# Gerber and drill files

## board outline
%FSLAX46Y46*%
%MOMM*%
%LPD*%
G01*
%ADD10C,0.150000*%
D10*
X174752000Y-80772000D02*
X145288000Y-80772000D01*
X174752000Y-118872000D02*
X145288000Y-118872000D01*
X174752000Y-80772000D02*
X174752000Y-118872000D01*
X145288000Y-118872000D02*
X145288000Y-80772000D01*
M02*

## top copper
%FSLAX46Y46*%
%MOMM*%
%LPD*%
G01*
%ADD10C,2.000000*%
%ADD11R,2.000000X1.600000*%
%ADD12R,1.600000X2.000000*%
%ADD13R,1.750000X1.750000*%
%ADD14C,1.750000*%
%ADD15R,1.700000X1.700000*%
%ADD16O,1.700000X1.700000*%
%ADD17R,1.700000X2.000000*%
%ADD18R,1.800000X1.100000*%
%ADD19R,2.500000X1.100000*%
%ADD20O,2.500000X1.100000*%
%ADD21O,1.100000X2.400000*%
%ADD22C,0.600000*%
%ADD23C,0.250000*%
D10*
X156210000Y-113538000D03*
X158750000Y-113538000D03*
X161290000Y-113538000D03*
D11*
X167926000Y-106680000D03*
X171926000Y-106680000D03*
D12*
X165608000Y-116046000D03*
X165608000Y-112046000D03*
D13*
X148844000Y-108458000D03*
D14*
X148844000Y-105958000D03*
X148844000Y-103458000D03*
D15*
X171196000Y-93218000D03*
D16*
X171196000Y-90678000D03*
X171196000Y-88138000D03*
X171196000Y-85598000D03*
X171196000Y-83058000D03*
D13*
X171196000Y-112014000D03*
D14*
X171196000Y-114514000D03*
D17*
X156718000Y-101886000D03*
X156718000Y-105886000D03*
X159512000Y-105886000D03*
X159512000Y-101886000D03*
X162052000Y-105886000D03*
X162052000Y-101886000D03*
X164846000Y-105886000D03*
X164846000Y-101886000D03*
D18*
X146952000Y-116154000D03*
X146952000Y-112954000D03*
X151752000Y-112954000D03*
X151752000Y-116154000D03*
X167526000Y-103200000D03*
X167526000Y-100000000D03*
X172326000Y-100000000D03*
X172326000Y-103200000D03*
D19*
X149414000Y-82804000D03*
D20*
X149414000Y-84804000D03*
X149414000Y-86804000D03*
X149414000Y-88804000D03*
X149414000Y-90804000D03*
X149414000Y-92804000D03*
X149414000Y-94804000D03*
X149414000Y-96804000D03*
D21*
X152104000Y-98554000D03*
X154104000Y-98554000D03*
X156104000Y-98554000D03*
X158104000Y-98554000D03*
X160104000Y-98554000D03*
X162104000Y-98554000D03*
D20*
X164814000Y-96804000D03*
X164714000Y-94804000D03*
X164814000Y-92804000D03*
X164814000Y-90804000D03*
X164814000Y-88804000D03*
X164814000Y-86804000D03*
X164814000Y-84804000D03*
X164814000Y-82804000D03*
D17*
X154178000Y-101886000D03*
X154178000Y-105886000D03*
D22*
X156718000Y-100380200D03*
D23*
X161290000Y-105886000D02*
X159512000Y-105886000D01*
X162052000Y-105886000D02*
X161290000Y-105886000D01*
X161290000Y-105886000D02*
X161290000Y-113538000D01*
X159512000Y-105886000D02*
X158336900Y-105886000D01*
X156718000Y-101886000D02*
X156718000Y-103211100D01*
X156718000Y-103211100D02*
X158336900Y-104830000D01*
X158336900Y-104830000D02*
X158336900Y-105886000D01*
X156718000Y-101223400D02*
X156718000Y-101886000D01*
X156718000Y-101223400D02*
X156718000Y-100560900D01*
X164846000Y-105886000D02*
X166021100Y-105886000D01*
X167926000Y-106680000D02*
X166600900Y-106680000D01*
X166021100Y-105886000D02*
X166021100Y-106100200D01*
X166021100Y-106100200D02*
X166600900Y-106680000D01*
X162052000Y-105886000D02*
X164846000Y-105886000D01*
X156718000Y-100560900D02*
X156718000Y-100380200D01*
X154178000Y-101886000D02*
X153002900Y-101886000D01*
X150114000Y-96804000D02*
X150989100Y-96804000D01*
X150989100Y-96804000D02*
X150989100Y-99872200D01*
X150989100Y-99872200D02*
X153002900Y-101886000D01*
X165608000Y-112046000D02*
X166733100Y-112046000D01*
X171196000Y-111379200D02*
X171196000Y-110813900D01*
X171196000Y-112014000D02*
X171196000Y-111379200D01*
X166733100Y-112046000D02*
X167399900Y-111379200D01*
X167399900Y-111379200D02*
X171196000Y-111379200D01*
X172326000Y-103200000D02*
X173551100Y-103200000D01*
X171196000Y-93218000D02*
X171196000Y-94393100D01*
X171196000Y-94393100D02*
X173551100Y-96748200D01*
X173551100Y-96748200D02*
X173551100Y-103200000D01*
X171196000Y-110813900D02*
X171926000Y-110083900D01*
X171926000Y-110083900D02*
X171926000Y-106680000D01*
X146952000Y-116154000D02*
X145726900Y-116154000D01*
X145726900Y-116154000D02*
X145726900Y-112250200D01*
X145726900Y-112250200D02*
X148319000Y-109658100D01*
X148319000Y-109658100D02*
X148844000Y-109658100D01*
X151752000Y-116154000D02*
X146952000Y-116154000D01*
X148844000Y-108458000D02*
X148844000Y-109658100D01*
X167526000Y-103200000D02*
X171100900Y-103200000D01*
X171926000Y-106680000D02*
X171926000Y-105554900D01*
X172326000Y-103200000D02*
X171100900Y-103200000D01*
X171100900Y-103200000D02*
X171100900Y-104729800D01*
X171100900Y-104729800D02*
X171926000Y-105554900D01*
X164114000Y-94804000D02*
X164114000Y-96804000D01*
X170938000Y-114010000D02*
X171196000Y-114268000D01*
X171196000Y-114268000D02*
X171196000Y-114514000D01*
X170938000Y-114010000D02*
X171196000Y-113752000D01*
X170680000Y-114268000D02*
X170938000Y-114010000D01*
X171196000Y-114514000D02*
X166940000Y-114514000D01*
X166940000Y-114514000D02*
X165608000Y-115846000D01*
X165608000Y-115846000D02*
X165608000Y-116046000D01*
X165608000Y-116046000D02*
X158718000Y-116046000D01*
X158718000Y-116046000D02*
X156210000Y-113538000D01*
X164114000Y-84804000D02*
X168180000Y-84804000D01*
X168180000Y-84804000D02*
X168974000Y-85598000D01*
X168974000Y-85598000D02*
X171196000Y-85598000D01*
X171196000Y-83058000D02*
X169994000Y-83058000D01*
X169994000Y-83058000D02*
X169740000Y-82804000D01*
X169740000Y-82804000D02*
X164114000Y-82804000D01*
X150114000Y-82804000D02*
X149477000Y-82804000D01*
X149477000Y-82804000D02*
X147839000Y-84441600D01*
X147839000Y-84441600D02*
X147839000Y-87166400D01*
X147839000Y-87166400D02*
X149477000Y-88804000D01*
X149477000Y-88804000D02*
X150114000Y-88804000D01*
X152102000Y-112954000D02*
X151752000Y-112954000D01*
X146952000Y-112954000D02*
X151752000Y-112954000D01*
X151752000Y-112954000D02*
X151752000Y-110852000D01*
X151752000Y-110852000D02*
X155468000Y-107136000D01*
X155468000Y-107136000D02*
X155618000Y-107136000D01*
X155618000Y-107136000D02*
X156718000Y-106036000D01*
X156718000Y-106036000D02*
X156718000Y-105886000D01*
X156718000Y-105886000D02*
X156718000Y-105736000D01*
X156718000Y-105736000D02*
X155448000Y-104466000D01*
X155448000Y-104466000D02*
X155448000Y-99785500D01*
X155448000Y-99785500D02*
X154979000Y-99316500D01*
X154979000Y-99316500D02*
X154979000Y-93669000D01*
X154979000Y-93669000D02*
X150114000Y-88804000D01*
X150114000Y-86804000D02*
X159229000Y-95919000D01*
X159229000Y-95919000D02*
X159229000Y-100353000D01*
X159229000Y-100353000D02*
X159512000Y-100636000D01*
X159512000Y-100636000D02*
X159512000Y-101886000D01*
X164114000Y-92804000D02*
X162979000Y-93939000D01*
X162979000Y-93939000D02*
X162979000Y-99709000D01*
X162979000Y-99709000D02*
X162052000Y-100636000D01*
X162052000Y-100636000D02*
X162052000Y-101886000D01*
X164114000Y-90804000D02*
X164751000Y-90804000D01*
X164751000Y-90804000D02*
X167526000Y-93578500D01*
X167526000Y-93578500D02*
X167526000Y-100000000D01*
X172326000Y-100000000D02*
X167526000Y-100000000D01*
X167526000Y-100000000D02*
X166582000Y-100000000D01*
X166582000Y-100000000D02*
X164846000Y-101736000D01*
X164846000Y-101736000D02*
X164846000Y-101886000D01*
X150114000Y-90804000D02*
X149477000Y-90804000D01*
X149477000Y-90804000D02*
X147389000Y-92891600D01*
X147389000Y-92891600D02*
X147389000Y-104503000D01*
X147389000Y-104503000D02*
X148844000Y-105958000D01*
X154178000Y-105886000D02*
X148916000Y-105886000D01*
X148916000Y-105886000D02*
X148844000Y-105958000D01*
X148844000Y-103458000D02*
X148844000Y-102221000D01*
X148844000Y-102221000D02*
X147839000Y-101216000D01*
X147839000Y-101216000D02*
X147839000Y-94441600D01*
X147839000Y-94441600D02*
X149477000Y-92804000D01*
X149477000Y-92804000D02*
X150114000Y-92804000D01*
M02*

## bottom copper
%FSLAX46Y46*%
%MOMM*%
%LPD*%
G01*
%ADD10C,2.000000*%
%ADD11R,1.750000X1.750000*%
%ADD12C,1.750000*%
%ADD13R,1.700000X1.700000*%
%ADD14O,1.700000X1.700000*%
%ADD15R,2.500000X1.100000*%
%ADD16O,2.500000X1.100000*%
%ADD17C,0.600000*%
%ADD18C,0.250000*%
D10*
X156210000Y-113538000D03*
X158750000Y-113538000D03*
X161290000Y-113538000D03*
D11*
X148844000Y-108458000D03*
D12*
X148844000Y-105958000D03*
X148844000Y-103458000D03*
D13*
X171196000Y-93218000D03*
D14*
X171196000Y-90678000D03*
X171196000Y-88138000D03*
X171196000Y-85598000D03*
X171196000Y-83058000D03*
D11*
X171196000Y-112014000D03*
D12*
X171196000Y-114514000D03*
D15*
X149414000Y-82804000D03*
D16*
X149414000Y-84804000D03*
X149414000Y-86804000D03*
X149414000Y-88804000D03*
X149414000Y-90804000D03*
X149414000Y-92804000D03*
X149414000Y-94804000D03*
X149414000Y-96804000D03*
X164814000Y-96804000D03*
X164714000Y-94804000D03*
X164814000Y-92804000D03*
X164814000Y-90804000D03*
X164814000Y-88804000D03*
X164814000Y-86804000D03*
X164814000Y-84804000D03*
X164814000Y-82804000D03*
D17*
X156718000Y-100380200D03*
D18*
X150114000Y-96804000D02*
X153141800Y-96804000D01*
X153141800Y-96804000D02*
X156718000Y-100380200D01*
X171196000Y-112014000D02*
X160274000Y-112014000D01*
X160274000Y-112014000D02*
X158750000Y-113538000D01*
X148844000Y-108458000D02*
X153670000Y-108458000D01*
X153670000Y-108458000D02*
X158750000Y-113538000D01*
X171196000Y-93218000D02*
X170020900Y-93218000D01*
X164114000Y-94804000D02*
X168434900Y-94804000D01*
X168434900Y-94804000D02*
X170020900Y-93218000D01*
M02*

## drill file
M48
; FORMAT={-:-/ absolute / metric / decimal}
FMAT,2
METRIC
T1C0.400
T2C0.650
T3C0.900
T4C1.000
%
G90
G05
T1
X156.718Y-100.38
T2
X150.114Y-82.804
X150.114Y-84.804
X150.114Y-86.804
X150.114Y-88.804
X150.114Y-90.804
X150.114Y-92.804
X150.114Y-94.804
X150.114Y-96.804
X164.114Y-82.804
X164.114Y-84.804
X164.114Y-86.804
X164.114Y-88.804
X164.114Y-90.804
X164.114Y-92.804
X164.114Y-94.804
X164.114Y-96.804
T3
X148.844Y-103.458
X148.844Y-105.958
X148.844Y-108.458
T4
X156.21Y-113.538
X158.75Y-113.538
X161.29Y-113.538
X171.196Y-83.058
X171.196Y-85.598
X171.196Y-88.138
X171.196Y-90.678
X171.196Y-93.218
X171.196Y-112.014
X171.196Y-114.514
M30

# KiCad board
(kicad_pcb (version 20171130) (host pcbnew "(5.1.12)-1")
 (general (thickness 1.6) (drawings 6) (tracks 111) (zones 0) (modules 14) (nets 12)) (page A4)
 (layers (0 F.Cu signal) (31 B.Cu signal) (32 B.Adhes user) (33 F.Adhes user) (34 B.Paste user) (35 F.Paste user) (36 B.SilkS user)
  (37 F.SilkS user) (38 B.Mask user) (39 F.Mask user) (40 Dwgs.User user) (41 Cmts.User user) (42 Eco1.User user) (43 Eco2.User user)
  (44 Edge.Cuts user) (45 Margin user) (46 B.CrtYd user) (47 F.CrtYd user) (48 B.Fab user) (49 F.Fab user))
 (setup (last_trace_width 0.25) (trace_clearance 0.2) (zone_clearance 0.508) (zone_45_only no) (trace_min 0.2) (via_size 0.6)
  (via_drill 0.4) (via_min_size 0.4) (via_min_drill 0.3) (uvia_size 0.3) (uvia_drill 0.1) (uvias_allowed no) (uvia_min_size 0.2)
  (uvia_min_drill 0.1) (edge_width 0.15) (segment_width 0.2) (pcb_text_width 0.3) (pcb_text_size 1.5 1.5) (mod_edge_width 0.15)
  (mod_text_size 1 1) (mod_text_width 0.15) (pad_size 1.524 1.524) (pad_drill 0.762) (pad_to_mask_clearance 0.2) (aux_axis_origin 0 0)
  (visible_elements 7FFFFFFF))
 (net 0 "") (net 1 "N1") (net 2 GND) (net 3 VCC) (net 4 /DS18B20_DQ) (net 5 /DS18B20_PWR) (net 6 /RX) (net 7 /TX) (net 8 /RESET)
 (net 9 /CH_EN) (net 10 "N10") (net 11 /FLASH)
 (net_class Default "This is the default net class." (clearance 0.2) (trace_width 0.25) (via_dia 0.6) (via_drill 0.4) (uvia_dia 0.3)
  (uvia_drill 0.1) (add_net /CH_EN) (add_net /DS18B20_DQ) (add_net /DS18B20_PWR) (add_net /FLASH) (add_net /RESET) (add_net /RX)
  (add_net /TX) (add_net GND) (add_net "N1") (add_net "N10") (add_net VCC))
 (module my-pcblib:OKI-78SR (layer F.Cu) (at 158.75 113.538)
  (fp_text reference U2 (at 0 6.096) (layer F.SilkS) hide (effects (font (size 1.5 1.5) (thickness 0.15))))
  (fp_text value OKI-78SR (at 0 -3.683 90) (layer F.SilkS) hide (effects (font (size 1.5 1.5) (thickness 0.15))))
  (pad 1 thru_hole circle (at -2.54 0) (size 2 2) (drill 1) (layers *.Cu *.Mask F.SilkS) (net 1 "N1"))
  (pad 2 thru_hole circle (at 0 0) (size 2 2) (drill 1) (layers *.Cu *.Mask F.SilkS) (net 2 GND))
  (pad 3 thru_hole circle (at 2.54 0) (size 2 2) (drill 1) (layers *.Cu *.Mask F.SilkS) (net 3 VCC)))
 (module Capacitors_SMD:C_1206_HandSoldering (layer F.Cu) (at 169.926 106.68)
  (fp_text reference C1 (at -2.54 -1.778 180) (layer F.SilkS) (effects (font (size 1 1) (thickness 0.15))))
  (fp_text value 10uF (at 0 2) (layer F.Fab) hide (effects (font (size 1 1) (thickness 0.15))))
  (pad 1 smd rect (at -2 0) (size 2 1.6) (layers F.Cu F.Paste F.Mask) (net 3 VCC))
  (pad 2 smd rect (at 2 0) (size 2 1.6) (layers F.Cu F.Paste F.Mask) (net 2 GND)))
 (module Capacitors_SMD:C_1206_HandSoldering (layer F.Cu) (at 165.608 114.046 90)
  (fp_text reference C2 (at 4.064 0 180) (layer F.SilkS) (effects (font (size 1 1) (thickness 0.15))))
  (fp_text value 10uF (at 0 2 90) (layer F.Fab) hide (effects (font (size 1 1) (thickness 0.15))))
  (pad 1 smd rect (at -2 0 90) (size 2 1.6) (layers F.Cu F.Paste F.Mask) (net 1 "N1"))
  (pad 2 smd rect (at 2 0 90) (size 2 1.6) (layers F.Cu F.Paste F.Mask) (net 2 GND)))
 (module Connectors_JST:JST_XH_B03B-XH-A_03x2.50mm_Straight (layer F.Cu) (at 148.844 108.458 90)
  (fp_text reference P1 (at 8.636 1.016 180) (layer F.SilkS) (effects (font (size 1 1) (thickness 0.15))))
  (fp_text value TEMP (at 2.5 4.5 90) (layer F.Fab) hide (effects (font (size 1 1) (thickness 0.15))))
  (pad 1 thru_hole rect (at 0 0 90) (size 1.75 1.75) (drill 0.9) (layers *.Cu *.Mask) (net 2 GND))
  (pad 2 thru_hole circle (at 2.5 0 90) (size 1.75 1.75) (drill 0.9) (layers *.Cu *.Mask) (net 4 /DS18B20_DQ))
  (pad 3 thru_hole circle (at 5 0 90) (size 1.75 1.75) (drill 0.9) (layers *.Cu *.Mask) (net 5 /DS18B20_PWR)))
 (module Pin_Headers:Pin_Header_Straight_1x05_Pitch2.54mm (layer F.Cu) (at 171.196 93.218 180)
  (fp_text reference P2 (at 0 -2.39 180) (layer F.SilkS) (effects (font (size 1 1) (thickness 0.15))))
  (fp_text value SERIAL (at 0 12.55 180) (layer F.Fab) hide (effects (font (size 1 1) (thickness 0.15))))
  (pad 1 thru_hole rect (at 0 0 180) (size 1.7 1.7) (drill 1) (layers *.Cu *.Mask) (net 2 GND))
  (pad 2 thru_hole oval (at 0 2.54 180) (size 1.7 1.7) (drill 1) (layers *.Cu *.Mask))
  (pad 3 thru_hole oval (at 0 5.08 180) (size 1.7 1.7) (drill 1) (layers *.Cu *.Mask))
  (pad 4 thru_hole oval (at 0 7.62 180) (size 1.7 1.7) (drill 1) (layers *.Cu *.Mask) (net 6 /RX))
  (pad 5 thru_hole oval (at 0 10.16 180) (size 1.7 1.7) (drill 1) (layers *.Cu *.Mask) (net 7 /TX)))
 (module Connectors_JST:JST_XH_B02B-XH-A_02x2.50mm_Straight (layer F.Cu) (at 171.196 112.014 270)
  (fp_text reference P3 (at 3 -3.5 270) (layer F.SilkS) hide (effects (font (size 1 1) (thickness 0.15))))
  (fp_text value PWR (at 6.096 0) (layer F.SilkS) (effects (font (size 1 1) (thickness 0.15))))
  (pad 1 thru_hole rect (at 0 0 270) (size 1.75 1.75) (drill 1) (layers *.Cu *.Mask) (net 2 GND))
  (pad 2 thru_hole circle (at 2.5 0 270) (size 1.75 1.75) (drill 1) (layers *.Cu *.Mask) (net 1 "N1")))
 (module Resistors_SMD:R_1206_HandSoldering (layer F.Cu) (at 156.718 103.886 270)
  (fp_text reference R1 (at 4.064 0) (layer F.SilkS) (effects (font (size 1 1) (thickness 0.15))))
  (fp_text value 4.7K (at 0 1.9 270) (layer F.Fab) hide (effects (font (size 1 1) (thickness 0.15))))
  (pad 1 smd rect (at -2 0 270) (size 2 1.7) (layers F.Cu F.Paste F.Mask) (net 3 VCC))
  (pad 2 smd rect (at 2 0 270) (size 2 1.7) (layers F.Cu F.Paste F.Mask) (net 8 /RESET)))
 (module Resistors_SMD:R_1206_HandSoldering (layer F.Cu) (at 159.512 103.886 90)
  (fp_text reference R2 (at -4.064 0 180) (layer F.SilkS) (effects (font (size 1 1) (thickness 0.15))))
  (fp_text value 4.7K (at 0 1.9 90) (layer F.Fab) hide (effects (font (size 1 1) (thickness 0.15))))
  (pad 1 smd rect (at -2 0 90) (size 2 1.7) (layers F.Cu F.Paste F.Mask) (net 3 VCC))
  (pad 2 smd rect (at 2 0 90) (size 2 1.7) (layers F.Cu F.Paste F.Mask) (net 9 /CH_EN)))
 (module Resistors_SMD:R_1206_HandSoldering (layer F.Cu) (at 162.052 103.886 90)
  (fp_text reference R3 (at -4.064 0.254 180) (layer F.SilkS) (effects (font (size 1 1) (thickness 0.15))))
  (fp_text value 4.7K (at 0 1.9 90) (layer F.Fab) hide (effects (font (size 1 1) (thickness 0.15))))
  (pad 1 smd rect (at -2 0 90) (size 2 1.7) (layers F.Cu F.Paste F.Mask) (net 3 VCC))
  (pad 2 smd rect (at 2 0 90) (size 2 1.7) (layers F.Cu F.Paste F.Mask) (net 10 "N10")))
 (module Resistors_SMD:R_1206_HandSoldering (layer F.Cu) (at 164.846 103.886 90)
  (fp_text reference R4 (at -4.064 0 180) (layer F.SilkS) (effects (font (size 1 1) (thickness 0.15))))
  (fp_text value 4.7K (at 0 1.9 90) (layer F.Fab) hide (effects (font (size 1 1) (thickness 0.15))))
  (pad 1 smd rect (at -2 0 90) (size 2 1.7) (layers F.Cu F.Paste F.Mask) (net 3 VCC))
  (pad 2 smd rect (at 2 0 90) (size 2 1.7) (layers F.Cu F.Paste F.Mask) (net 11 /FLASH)))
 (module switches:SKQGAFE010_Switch (layer F.Cu) (at 149.352 114.554)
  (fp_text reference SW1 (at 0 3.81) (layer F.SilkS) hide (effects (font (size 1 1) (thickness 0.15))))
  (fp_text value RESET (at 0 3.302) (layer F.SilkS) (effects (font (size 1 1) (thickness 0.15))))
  (pad 3 smd rect (at -2.4 1.6) (size 1.8 1.1) (layers F.Cu F.Paste F.Mask) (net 2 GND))
  (pad 1 smd rect (at -2.4 -1.6) (size 1.8 1.1) (layers F.Cu F.Paste F.Mask) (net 8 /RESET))
  (pad 2 smd rect (at 2.4 -1.6) (size 1.8 1.1) (layers F.Cu F.Paste F.Mask) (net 8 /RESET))
  (pad 4 smd rect (at 2.4 1.6) (size 1.8 1.1) (layers F.Cu F.Paste F.Mask) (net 2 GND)))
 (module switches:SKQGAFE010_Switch (layer F.Cu) (at 169.926 101.6)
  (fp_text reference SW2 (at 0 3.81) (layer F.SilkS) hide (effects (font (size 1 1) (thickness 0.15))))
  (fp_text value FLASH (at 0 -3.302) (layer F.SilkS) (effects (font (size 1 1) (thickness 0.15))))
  (pad 3 smd rect (at -2.4 1.6) (size 1.8 1.1) (layers F.Cu F.Paste F.Mask) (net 2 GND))
  (pad 1 smd rect (at -2.4 -1.6) (size 1.8 1.1) (layers F.Cu F.Paste F.Mask) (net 11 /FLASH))
  (pad 2 smd rect (at 2.4 -1.6) (size 1.8 1.1) (layers F.Cu F.Paste F.Mask) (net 11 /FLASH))
  (pad 4 smd rect (at 2.4 1.6) (size 1.8 1.1) (layers F.Cu F.Paste F.Mask) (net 2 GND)))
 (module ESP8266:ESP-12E (layer F.Cu) (at 150.114 82.804)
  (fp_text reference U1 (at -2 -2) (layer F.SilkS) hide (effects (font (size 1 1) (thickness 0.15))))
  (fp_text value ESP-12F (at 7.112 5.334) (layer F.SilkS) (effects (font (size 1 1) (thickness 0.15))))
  (pad 1 thru_hole rect (at 0 0) (size 2.5 1.1) (drill 0.65 (offset -0.7 0)) (layers *.Cu *.Mask F.SilkS) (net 8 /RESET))
  (pad 2 thru_hole oval (at 0 2) (size 2.5 1.1) (drill 0.65 (offset -0.7 0)) (layers *.Cu *.Mask F.SilkS))
  (pad 3 thru_hole oval (at 0 4) (size 2.5 1.1) (drill 0.65 (offset -0.7 0)) (layers *.Cu *.Mask F.SilkS) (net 9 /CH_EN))
  (pad 4 thru_hole oval (at 0 6) (size 2.5 1.1) (drill 0.65 (offset -0.7 0)) (layers *.Cu *.Mask F.SilkS) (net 8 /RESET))
  (pad 5 thru_hole oval (at 0 8) (size 2.5 1.1) (drill 0.65 (offset -0.7 0)) (layers *.Cu *.Mask F.SilkS) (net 4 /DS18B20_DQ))
  (pad 6 thru_hole oval (at 0 10) (size 2.5 1.1) (drill 0.65 (offset -0.7 0)) (layers *.Cu *.Mask F.SilkS) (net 5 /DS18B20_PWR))
  (pad 7 thru_hole oval (at 0 12) (size 2.5 1.1) (drill 0.65 (offset -0.7 0)) (layers *.Cu *.Mask F.SilkS))
  (pad 8 thru_hole oval (at 0 14) (size 2.5 1.1) (drill 0.65 (offset -0.7 0)) (layers *.Cu *.Mask F.SilkS) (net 3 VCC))
  (pad 9 smd oval (at 1.99 15.75 90) (size 2.4 1.1) (layers F.Cu F.Paste F.Mask))
  (pad 10 smd oval (at 3.99 15.75 90) (size 2.4 1.1) (layers F.Cu F.Paste F.Mask))
  (pad 11 smd oval (at 5.99 15.75 90) (size 2.4 1.1) (layers F.Cu F.Paste F.Mask))
  (pad 12 smd oval (at 7.99 15.75 90) (size 2.4 1.1) (layers F.Cu F.Paste F.Mask))
  (pad 13 smd oval (at 9.99 15.75 90) (size 2.4 1.1) (layers F.Cu F.Paste F.Mask))
  (pad 14 smd oval (at 11.99 15.75 90) (size 2.4 1.1) (layers F.Cu F.Paste F.Mask))
  (pad 15 thru_hole oval (at 14 14) (size 2.5 1.1) (drill 0.65 (offset 0.7 0)) (layers *.Cu *.Mask F.SilkS) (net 2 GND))
  (pad 16 thru_hole oval (at 14 12) (size 2.5 1.1) (drill 0.65 (offset 0.6 0)) (layers *.Cu *.Mask F.SilkS) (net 2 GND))
  (pad 17 thru_hole oval (at 14 10) (size 2.5 1.1) (drill 0.65 (offset 0.7 0)) (layers *.Cu *.Mask F.SilkS) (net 10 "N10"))
  (pad 18 thru_hole oval (at 14 8) (size 2.5 1.1) (drill 0.65 (offset 0.7 0)) (layers *.Cu *.Mask F.SilkS) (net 11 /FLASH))
  (pad 19 thru_hole oval (at 14 6) (size 2.5 1.1) (drill 0.65 (offset 0.7 0)) (layers *.Cu *.Mask F.SilkS))
  (pad 20 thru_hole oval (at 14 4) (size 2.5 1.1) (drill 0.65 (offset 0.7 0)) (layers *.Cu *.Mask F.SilkS))
  (pad 21 thru_hole oval (at 14 2) (size 2.5 1.1) (drill 0.65 (offset 0.7 0)) (layers *.Cu *.Mask F.SilkS) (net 6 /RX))
  (pad 22 thru_hole oval (at 14 0) (size 2.5 1.1) (drill 0.65 (offset 0.7 0)) (layers *.Cu *.Mask F.SilkS) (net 7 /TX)))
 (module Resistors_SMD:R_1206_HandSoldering (layer F.Cu) (at 154.178 103.886 270)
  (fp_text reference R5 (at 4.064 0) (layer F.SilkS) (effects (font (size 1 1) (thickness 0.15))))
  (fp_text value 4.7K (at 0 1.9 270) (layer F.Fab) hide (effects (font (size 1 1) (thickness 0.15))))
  (pad 1 smd rect (at -2 0 270) (size 2 1.7) (layers F.Cu F.Paste F.Mask) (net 3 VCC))
  (pad 2 smd rect (at 2 0 270) (size 2 1.7) (layers F.Cu F.Paste F.Mask) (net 4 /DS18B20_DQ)))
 (gr_line (start 174.752 80.772) (end 145.288 80.772) (angle 90) (layer Edge.Cuts) (width 0.15))
 (gr_line (start 174.752 118.872) (end 145.288 118.872) (angle 90) (layer Edge.Cuts) (width 0.15))
 (gr_line (start 174.752 80.772) (end 174.752 118.872) (angle 90) (layer Edge.Cuts) (width 0.15))
 (gr_line (start 145.288 118.872) (end 145.288 80.772) (angle 90) (layer Edge.Cuts) (width 0.15))
 (segment (start 161.29 105.886) (end 159.512 105.886) (width 0.25) (layer F.Cu) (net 3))
 (segment (start 162.052 105.886) (end 161.29 105.886) (width 0.25) (layer F.Cu) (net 3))
 (segment (start 161.29 105.886) (end 161.29 113.538) (width 0.25) (layer F.Cu) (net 3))
 (segment (start 159.512 105.886) (end 158.3369 105.886) (width 0.25) (layer F.Cu) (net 3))
 (segment (start 156.718 101.886) (end 156.718 103.2111) (width 0.25) (layer F.Cu) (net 3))
 (segment (start 156.718 103.2111) (end 158.3369 104.83) (width 0.25) (layer F.Cu) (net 3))
 (segment (start 158.3369 104.83) (end 158.3369 105.886) (width 0.25) (layer F.Cu) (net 3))
 (segment (start 156.718 101.2234) (end 156.718 101.886) (width 0.25) (layer F.Cu) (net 3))
 (segment (start 156.718 101.2234) (end 156.718 100.5609) (width 0.25) (layer F.Cu) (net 3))
 (segment (start 164.846 105.886) (end 166.0211 105.886) (width 0.25) (layer F.Cu) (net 3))
 (segment (start 167.926 106.68) (end 166.6009 106.68) (width 0.25) (layer F.Cu) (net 3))
 (segment (start 166.0211 105.886) (end 166.0211 106.1002) (width 0.25) (layer F.Cu) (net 3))
 (segment (start 166.0211 106.1002) (end 166.6009 106.68) (width 0.25) (layer F.Cu) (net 3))
 (segment (start 162.052 105.886) (end 164.846 105.886) (width 0.25) (layer F.Cu) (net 3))
 (segment (start 156.718 100.5609) (end 156.718 100.3802) (width 0.25) (layer F.Cu) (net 3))
 (segment (start 150.114 96.804) (end 153.1418 96.804) (width 0.25) (layer B.Cu) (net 3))
 (segment (start 153.1418 96.804) (end 156.718 100.3802) (width 0.25) (layer B.Cu) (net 3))
 (segment (start 154.178 101.886) (end 153.0029 101.886) (width 0.25) (layer F.Cu) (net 3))
 (segment (start 150.114 96.804) (end 150.9891 96.804) (width 0.25) (layer F.Cu) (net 3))
 (segment (start 150.9891 96.804) (end 150.9891 99.8722) (width 0.25) (layer F.Cu) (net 3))
 (segment (start 150.9891 99.8722) (end 153.0029 101.886) (width 0.25) (layer F.Cu) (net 3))
 (via (at 156.718 100.3802) (size 0.6) (layers F.Cu B.Cu) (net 3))
 (segment (start 171.196 112.014) (end 160.274 112.014) (width 0.25) (layer B.Cu) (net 2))
 (segment (start 160.274 112.014) (end 158.75 113.538) (width 0.25) (layer B.Cu) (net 2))
 (segment (start 165.608 112.046) (end 166.7331 112.046) (width 0.25) (layer F.Cu) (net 2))
 (segment (start 171.196 111.3792) (end 171.196 110.8139) (width 0.25) (layer F.Cu) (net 2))
 (segment (start 171.196 112.014) (end 171.196 111.3792) (width 0.25) (layer F.Cu) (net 2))
 (segment (start 166.7331 112.046) (end 167.3999 111.3792) (width 0.25) (layer F.Cu) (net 2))
 (segment (start 167.3999 111.3792) (end 171.196 111.3792) (width 0.25) (layer F.Cu) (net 2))
 (segment (start 148.844 108.458) (end 153.67 108.458) (width 0.25) (layer B.Cu) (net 2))
 (segment (start 153.67 108.458) (end 158.75 113.538) (width 0.25) (layer B.Cu) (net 2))
 (segment (start 172.326 103.2) (end 173.5511 103.2) (width 0.25) (layer F.Cu) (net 2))
 (segment (start 171.196 93.218) (end 171.196 94.3931) (width 0.25) (layer F.Cu) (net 2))
 (segment (start 171.196 94.3931) (end 173.5511 96.7482) (width 0.25) (layer F.Cu) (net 2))
 (segment (start 173.5511 96.7482) (end 173.5511 103.2) (width 0.25) (layer F.Cu) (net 2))
 (segment (start 171.196 110.8139) (end 171.926 110.0839) (width 0.25) (layer F.Cu) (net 2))
 (segment (start 171.926 110.0839) (end 171.926 106.68) (width 0.25) (layer F.Cu) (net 2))
 (segment (start 146.952 116.154) (end 145.7269 116.154) (width 0.25) (layer F.Cu) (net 2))
 (segment (start 145.7269 116.154) (end 145.7269 112.2502) (width 0.25) (layer F.Cu) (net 2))
 (segment (start 145.7269 112.2502) (end 148.319 109.6581) (width 0.25) (layer F.Cu) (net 2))
 (segment (start 148.319 109.6581) (end 148.844 109.6581) (width 0.25) (layer F.Cu) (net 2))
 (segment (start 151.752 116.154) (end 146.952 116.154) (width 0.25) (layer F.Cu) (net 2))
 (segment (start 148.844 108.458) (end 148.844 109.6581) (width 0.25) (layer F.Cu) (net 2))
 (segment (start 167.526 103.2) (end 171.1009 103.2) (width 0.25) (layer F.Cu) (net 2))
 (segment (start 171.926 106.68) (end 171.926 105.5549) (width 0.25) (layer F.Cu) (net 2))
 (segment (start 172.326 103.2) (end 171.1009 103.2) (width 0.25) (layer F.Cu) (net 2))
 (segment (start 171.1009 103.2) (end 171.1009 104.7298) (width 0.25) (layer F.Cu) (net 2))
 (segment (start 171.1009 104.7298) (end 171.926 105.5549) (width 0.25) (layer F.Cu) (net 2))
 (segment (start 171.196 93.218) (end 170.0209 93.218) (width 0.25) (layer B.Cu) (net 2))
 (segment (start 164.114 94.804) (end 168.4349 94.804) (width 0.25) (layer B.Cu) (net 2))
 (segment (start 168.4349 94.804) (end 170.0209 93.218) (width 0.25) (layer B.Cu) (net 2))
 (segment (start 164.114 94.804) (end 164.114 96.804) (width 0.25) (layer F.Cu) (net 2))
 (segment (start 170.938 114.01) (end 171.196 114.268) (width 0.25) (layer F.Cu) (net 1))
 (segment (start 171.196 114.268) (end 171.196 114.514) (width 0.25) (layer F.Cu) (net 1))
 (segment (start 170.938 114.01) (end 171.196 113.752) (width 0.25) (layer F.Cu) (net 1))
 (segment (start 170.68 114.268) (end 170.938 114.01) (width 0.25) (layer F.Cu) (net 1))
 (segment (start 171.196 114.514) (end 166.94 114.514) (width 0.25) (layer F.Cu) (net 1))
 (segment (start 166.94 114.514) (end 165.608 115.846) (width 0.25) (layer F.Cu) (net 1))
 (segment (start 165.608 115.846) (end 165.608 116.046) (width 0.25) (layer F.Cu) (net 1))
 (segment (start 165.608 116.046) (end 158.718 116.046) (width 0.25) (layer F.Cu) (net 1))
 (segment (start 158.718 116.046) (end 156.21 113.538) (width 0.25) (layer F.Cu) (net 1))
 (segment (start 164.114 84.804) (end 168.18 84.804) (width 0.25) (layer F.Cu) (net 6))
 (segment (start 168.18 84.804) (end 168.974 85.598) (width 0.25) (layer F.Cu) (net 6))
 (segment (start 168.974 85.598) (end 171.196 85.598) (width 0.25) (layer F.Cu) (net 6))
 (segment (start 171.196 83.058) (end 169.994 83.058) (width 0.25) (layer F.Cu) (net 7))
 (segment (start 169.994 83.058) (end 169.74 82.804) (width 0.25) (layer F.Cu) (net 7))
 (segment (start 169.74 82.804) (end 164.114 82.804) (width 0.25) (layer F.Cu) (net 7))
 (segment (start 150.114 82.804) (end 149.477 82.804) (width 0.25) (layer F.Cu) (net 8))
 (segment (start 149.477 82.804) (end 147.839 84.4416) (width 0.25) (layer F.Cu) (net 8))
 (segment (start 147.839 84.4416) (end 147.839 87.1664) (width 0.25) (layer F.Cu) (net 8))
 (segment (start 147.839 87.1664) (end 149.477 88.804) (width 0.25) (layer F.Cu) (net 8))
 (segment (start 149.477 88.804) (end 150.114 88.804) (width 0.25) (layer F.Cu) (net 8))
 (segment (start 152.102 112.954) (end 151.752 112.954) (width 0.25) (layer F.Cu) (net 8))
 (segment (start 146.952 112.954) (end 151.752 112.954) (width 0.25) (layer F.Cu) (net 8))
 (segment (start 151.752 112.954) (end 151.752 110.852) (width 0.25) (layer F.Cu) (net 8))
 (segment (start 151.752 110.852) (end 155.468 107.136) (width 0.25) (layer F.Cu) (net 8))
 (segment (start 155.468 107.136) (end 155.618 107.136) (width 0.25) (layer F.Cu) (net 8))
 (segment (start 155.618 107.136) (end 156.718 106.036) (width 0.25) (layer F.Cu) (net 8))
 (segment (start 156.718 106.036) (end 156.718 105.886) (width 0.25) (layer F.Cu) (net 8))
 (segment (start 156.718 105.886) (end 156.718 105.736) (width 0.25) (layer F.Cu) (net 8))
 (segment (start 156.718 105.736) (end 155.448 104.466) (width 0.25) (layer F.Cu) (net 8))
 (segment (start 155.448 104.466) (end 155.448 99.7855) (width 0.25) (layer F.Cu) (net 8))
 (segment (start 155.448 99.7855) (end 154.979 99.3165) (width 0.25) (layer F.Cu) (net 8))
 (segment (start 154.979 99.3165) (end 154.979 93.669) (width 0.25) (layer F.Cu) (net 8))
 (segment (start 154.979 93.669) (end 150.114 88.804) (width 0.25) (layer F.Cu) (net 8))
 (segment (start 150.114 86.804) (end 159.229 95.919) (width 0.25) (layer F.Cu) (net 9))
 (segment (start 159.229 95.919) (end 159.229 100.353) (width 0.25) (layer F.Cu) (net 9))
 (segment (start 159.229 100.353) (end 159.512 100.636) (width 0.25) (layer F.Cu) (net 9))
 (segment (start 159.512 100.636) (end 159.512 101.886) (width 0.25) (layer F.Cu) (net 9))
 (segment (start 164.114 92.804) (end 162.979 93.939) (width 0.25) (layer F.Cu) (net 10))
 (segment (start 162.979 93.939) (end 162.979 99.709) (width 0.25) (layer F.Cu) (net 10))
 (segment (start 162.979 99.709) (end 162.052 100.636) (width 0.25) (layer F.Cu) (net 10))
 (segment (start 162.052 100.636) (end 162.052 101.886) (width 0.25) (layer F.Cu) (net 10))
 (segment (start 164.114 90.804) (end 164.751 90.804) (width 0.25) (layer F.Cu) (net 11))
 (segment (start 164.751 90.804) (end 167.526 93.5785) (width 0.25) (layer F.Cu) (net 11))
 (segment (start 167.526 93.5785) (end 167.526 100) (width 0.25) (layer F.Cu) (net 11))
 (segment (start 172.326 100) (end 167.526 100) (width 0.25) (layer F.Cu) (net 11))
 (segment (start 167.526 100) (end 166.582 100) (width 0.25) (layer F.Cu) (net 11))
 (segment (start 166.582 100) (end 164.846 101.736) (width 0.25) (layer F.Cu) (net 11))
 (segment (start 164.846 101.736) (end 164.846 101.886) (width 0.25) (layer F.Cu) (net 11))
 (segment (start 150.114 90.804) (end 149.477 90.804) (width 0.25) (layer F.Cu) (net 4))
 (segment (start 149.477 90.804) (end 147.389 92.8916) (width 0.25) (layer F.Cu) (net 4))
 (segment (start 147.389 92.8916) (end 147.389 104.503) (width 0.25) (layer F.Cu) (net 4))
 (segment (start 147.389 104.503) (end 148.844 105.958) (width 0.25) (layer F.Cu) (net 4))
 (segment (start 154.178 105.886) (end 148.916 105.886) (width 0.25) (layer F.Cu) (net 4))
 (segment (start 148.916 105.886) (end 148.844 105.958) (width 0.25) (layer F.Cu) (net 4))
 (segment (start 148.844 103.458) (end 148.844 102.221) (width 0.25) (layer F.Cu) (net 5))
 (segment (start 148.844 102.221) (end 147.839 101.216) (width 0.25) (layer F.Cu) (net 5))
 (segment (start 147.839 101.216) (end 147.839 94.4416) (width 0.25) (layer F.Cu) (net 5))
 (segment (start 147.839 94.4416) (end 149.477 92.804) (width 0.25) (layer F.Cu) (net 5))
 (segment (start 149.477 92.804) (end 150.114 92.804) (width 0.25) (layer F.Cu) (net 5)))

